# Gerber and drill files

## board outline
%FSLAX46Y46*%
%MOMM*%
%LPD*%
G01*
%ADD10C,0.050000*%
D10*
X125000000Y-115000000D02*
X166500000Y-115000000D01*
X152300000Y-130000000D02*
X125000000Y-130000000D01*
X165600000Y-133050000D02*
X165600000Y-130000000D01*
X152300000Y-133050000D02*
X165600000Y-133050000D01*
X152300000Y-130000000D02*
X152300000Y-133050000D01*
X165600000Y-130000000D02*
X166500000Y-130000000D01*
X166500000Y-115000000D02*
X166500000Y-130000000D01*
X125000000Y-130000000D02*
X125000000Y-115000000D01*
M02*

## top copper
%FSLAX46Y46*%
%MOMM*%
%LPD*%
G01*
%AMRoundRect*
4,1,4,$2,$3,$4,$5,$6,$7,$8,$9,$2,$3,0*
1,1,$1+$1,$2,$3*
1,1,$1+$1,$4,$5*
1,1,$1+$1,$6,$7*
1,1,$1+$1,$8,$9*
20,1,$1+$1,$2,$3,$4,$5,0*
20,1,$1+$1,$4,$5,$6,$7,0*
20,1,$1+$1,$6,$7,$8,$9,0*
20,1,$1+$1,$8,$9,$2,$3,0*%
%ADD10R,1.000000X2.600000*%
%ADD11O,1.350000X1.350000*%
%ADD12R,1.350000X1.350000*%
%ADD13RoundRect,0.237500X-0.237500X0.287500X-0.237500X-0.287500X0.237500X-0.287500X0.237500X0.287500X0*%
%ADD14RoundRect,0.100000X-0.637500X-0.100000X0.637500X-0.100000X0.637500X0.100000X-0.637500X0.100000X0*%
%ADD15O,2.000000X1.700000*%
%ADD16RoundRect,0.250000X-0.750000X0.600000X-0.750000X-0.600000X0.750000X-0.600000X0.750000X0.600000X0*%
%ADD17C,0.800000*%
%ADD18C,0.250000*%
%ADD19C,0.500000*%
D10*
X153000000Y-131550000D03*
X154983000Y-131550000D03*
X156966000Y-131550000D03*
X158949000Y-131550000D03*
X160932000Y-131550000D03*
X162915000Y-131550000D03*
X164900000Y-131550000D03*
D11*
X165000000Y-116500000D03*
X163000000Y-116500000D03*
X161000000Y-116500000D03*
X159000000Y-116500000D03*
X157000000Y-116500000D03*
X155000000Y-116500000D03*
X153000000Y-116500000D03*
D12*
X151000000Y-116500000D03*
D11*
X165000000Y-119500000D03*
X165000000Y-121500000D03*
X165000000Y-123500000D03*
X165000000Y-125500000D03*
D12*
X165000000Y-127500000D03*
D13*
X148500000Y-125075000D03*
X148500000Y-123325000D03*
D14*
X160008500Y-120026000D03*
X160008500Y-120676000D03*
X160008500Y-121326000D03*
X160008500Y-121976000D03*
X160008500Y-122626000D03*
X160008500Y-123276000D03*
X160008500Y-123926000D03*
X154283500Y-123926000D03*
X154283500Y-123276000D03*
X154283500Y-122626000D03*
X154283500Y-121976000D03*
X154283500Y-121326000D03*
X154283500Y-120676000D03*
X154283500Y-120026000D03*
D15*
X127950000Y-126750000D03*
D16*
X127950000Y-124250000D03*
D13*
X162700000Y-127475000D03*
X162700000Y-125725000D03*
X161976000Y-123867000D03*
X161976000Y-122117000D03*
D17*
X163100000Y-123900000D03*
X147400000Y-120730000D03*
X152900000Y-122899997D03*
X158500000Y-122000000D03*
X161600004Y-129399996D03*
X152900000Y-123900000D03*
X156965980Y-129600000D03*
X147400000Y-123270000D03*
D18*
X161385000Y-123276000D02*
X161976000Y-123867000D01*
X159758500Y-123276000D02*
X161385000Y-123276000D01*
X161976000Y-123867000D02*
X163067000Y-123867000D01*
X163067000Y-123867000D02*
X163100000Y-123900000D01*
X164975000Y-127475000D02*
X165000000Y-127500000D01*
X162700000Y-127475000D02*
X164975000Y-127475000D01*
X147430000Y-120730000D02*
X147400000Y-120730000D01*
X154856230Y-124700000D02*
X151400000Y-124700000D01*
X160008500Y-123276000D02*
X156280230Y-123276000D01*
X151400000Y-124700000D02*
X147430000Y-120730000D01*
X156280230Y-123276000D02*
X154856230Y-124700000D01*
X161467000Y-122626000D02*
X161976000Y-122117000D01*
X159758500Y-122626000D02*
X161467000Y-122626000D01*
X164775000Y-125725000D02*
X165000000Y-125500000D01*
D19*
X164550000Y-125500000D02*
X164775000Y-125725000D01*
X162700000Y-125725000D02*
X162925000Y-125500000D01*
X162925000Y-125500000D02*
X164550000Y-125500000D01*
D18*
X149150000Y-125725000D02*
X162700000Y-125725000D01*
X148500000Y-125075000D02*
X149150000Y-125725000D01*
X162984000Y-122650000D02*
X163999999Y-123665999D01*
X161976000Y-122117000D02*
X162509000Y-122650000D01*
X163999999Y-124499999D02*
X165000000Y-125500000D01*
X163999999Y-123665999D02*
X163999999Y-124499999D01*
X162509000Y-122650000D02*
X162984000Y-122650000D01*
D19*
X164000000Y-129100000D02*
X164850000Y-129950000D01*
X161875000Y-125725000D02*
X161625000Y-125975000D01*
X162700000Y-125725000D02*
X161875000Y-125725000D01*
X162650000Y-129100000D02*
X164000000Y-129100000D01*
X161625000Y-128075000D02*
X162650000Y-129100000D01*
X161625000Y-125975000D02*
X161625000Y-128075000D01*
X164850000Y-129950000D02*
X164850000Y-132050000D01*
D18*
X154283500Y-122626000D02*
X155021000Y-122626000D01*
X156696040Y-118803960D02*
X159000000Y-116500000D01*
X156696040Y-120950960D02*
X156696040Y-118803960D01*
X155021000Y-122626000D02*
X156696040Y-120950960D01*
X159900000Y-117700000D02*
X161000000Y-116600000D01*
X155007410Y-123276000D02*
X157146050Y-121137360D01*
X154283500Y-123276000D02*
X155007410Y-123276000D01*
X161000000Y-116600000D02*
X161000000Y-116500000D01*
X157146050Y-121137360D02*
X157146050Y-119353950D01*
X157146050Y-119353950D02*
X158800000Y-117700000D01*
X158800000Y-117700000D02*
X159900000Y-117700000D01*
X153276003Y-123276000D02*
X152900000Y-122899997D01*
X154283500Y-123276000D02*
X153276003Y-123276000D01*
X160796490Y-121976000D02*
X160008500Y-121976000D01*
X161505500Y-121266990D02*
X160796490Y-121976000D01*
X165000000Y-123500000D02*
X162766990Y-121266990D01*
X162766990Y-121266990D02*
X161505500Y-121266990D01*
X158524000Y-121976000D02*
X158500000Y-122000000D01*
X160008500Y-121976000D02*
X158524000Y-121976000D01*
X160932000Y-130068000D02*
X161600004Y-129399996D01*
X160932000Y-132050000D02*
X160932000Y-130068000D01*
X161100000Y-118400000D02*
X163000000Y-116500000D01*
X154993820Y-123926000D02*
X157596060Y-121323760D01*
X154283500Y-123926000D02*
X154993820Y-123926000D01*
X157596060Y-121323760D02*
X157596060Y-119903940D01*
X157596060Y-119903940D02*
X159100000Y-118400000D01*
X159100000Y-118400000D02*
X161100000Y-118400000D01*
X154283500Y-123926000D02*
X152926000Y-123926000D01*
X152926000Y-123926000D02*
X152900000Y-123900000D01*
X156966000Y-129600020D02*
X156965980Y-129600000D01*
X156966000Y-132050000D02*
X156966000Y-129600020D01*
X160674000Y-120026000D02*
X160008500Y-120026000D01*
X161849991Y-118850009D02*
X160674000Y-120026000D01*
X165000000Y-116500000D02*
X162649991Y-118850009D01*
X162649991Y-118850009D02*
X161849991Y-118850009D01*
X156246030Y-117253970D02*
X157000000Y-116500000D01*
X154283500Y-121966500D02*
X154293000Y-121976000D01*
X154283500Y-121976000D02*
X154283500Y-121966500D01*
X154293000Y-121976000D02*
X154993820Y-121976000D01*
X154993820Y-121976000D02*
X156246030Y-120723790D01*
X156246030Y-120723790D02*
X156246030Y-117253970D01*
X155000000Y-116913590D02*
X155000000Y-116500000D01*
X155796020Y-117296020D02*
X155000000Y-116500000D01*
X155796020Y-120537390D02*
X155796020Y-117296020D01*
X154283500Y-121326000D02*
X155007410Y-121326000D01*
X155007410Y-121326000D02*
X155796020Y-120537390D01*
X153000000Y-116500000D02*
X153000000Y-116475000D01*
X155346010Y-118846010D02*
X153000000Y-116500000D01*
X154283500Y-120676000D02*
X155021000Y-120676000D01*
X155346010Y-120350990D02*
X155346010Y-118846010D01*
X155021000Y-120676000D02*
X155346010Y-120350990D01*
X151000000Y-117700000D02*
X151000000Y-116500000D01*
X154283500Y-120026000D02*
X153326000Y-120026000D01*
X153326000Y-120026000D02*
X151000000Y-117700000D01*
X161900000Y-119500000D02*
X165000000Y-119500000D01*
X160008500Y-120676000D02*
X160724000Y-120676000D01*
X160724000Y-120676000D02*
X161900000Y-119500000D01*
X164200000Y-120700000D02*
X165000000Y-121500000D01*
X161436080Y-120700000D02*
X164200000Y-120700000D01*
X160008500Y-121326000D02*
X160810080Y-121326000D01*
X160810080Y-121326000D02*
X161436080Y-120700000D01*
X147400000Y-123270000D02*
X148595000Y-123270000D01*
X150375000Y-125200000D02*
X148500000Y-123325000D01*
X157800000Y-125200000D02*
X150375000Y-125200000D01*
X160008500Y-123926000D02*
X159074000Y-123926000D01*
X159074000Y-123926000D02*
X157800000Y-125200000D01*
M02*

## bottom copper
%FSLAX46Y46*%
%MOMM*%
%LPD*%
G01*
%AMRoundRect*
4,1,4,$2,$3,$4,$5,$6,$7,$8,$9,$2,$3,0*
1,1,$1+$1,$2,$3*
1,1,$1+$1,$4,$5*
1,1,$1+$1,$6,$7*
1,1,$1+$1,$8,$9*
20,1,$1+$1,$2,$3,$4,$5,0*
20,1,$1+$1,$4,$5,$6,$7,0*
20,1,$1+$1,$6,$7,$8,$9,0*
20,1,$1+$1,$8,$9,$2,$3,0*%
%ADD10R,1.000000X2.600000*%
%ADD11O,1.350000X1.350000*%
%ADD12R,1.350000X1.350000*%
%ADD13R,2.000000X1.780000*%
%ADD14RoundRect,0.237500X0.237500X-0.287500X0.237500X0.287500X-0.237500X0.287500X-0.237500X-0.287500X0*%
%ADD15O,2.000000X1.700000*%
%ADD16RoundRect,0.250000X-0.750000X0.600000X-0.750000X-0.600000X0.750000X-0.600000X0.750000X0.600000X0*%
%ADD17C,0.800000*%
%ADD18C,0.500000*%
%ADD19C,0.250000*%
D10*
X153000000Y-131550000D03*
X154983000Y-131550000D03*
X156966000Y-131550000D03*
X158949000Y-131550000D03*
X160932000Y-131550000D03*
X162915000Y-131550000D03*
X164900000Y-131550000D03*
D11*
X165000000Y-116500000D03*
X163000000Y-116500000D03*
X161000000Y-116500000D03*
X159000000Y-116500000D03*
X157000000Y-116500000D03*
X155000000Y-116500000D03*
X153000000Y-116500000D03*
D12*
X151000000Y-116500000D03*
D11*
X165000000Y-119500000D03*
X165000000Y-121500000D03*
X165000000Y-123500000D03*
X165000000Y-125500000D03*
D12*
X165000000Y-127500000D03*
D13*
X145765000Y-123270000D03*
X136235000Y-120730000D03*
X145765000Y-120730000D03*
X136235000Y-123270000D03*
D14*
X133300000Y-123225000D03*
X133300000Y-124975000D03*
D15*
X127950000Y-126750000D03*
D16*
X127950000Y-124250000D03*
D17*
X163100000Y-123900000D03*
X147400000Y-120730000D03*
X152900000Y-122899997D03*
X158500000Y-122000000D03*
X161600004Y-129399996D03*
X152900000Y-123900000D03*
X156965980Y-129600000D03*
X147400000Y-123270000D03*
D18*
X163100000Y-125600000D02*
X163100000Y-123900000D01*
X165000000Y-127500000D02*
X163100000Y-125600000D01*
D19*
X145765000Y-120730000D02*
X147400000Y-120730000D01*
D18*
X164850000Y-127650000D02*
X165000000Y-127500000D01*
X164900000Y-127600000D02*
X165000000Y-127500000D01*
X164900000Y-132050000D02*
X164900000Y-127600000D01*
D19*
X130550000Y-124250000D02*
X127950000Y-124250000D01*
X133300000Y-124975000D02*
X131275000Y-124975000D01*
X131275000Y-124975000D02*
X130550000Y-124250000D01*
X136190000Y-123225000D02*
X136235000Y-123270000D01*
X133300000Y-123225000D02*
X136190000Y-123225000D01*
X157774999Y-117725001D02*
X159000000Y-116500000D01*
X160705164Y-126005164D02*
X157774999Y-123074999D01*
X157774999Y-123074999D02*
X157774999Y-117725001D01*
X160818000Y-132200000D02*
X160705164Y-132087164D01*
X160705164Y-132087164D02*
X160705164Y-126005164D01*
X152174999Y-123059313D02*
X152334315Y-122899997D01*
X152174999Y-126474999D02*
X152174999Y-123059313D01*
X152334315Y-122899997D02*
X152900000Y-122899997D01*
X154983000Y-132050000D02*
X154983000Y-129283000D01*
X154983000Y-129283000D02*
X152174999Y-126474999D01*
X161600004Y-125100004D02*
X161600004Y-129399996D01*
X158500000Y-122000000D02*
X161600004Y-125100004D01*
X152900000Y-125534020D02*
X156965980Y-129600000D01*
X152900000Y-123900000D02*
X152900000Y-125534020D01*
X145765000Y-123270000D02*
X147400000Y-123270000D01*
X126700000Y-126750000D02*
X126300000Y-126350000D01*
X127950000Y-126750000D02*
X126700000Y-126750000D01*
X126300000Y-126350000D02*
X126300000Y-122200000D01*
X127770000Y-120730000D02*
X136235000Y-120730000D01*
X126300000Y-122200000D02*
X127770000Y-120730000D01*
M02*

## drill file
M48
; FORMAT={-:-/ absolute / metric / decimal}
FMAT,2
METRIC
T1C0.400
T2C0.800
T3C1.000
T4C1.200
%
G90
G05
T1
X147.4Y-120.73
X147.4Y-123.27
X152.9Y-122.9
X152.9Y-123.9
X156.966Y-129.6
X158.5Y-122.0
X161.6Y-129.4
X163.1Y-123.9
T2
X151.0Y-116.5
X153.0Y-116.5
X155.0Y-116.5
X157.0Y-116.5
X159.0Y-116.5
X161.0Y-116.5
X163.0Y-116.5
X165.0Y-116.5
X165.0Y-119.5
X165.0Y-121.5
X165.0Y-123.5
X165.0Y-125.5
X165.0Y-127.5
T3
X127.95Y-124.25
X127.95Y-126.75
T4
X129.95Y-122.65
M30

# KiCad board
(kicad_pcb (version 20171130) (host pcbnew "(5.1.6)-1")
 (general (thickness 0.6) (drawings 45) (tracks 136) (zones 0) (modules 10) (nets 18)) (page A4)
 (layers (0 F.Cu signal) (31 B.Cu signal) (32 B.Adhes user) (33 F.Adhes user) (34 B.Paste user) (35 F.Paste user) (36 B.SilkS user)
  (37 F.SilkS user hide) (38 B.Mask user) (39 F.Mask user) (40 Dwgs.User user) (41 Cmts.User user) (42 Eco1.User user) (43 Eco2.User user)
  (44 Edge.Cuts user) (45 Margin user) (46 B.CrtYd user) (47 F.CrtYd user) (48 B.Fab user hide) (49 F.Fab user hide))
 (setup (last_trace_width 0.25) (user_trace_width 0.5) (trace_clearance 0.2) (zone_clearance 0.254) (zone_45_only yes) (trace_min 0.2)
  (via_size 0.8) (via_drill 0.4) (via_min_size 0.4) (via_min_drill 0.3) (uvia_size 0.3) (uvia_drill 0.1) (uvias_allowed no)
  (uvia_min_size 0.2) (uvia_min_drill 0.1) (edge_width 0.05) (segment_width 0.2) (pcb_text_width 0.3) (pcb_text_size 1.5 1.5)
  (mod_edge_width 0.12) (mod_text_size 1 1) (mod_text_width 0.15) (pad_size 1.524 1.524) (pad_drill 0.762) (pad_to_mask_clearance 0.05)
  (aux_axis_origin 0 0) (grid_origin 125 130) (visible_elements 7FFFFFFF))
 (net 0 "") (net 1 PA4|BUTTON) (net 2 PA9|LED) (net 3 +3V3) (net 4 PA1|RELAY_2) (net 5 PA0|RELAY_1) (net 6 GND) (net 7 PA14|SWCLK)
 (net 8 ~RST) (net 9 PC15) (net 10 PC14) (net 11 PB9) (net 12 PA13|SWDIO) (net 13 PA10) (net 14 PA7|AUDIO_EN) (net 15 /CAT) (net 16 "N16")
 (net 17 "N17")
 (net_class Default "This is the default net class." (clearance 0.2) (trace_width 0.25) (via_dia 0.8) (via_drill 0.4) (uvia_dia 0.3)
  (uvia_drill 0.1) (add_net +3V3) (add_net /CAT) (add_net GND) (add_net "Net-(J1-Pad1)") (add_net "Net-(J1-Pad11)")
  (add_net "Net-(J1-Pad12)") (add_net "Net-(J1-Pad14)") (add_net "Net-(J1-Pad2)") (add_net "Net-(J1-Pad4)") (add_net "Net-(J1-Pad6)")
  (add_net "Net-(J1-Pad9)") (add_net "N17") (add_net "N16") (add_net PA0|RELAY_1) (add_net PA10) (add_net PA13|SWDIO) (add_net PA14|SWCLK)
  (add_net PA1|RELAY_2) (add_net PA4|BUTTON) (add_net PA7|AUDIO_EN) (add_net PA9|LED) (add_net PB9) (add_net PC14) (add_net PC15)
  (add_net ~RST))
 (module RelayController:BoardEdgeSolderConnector (layer F.Cu) (at 153 131.55)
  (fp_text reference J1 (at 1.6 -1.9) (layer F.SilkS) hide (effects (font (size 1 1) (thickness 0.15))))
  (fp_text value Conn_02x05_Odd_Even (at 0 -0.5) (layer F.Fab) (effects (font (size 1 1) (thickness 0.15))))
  (pad 1 smd rect (at 0 0) (size 1 2.6) (layers F.Cu F.Paste F.Mask))
  (pad 2 smd rect (at 1.983 0) (size 1 2.6) (layers F.Cu F.Paste F.Mask))
  (pad 3 smd rect (at 3.966 0) (size 1 2.6) (layers F.Cu F.Paste F.Mask) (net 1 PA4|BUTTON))
  (pad 4 smd rect (at 5.949 0) (size 1 2.6) (layers F.Cu F.Paste F.Mask))
  (pad 5 smd rect (at 7.932 0) (size 1 2.6) (layers F.Cu F.Paste F.Mask) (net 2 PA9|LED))
  (pad 6 smd rect (at 9.915 0) (size 1 2.6) (layers F.Cu F.Paste F.Mask))
  (pad 7 smd rect (at 11.9 0) (size 1 2.6) (layers F.Cu F.Paste F.Mask) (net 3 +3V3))
  (pad 14 smd rect (at 0 0) (size 1 2.6) (layers B.Cu B.Paste B.Mask))
  (pad 13 smd rect (at 1.983 0) (size 1 2.6) (layers B.Cu B.Paste B.Mask) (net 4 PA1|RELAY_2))
  (pad 12 smd rect (at 3.966 0) (size 1 2.6) (layers B.Cu B.Paste B.Mask))
  (pad 11 smd rect (at 5.949 0) (size 1 2.6) (layers B.Cu B.Paste B.Mask))
  (pad 10 smd rect (at 7.932 0) (size 1 2.6) (layers B.Cu B.Paste B.Mask) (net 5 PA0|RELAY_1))
  (pad 9 smd rect (at 9.915 0) (size 1 2.6) (layers B.Cu B.Paste B.Mask))
  (pad 8 smd rect (at 11.9 0) (size 1 2.6) (layers B.Cu B.Paste B.Mask) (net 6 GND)))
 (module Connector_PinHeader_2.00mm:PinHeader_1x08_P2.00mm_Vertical (layer F.Cu) (at 151 116.5 90)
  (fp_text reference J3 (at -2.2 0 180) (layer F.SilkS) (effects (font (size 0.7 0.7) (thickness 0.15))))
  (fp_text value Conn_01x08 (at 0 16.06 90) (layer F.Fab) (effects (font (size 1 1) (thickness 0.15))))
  (pad 8 thru_hole oval (at 0 14 90) (size 1.35 1.35) (drill 0.8) (layers *.Cu *.Mask) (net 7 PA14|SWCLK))
  (pad 7 thru_hole oval (at 0 12 90) (size 1.35 1.35) (drill 0.8) (layers *.Cu *.Mask) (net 1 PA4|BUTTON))
  (pad 6 thru_hole oval (at 0 10 90) (size 1.35 1.35) (drill 0.8) (layers *.Cu *.Mask) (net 4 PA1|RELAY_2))
  (pad 5 thru_hole oval (at 0 8 90) (size 1.35 1.35) (drill 0.8) (layers *.Cu *.Mask) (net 5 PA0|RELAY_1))
  (pad 4 thru_hole oval (at 0 6 90) (size 1.35 1.35) (drill 0.8) (layers *.Cu *.Mask) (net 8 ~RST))
  (pad 3 thru_hole oval (at 0 4 90) (size 1.35 1.35) (drill 0.8) (layers *.Cu *.Mask) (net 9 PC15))
  (pad 2 thru_hole oval (at 0 2 90) (size 1.35 1.35) (drill 0.8) (layers *.Cu *.Mask) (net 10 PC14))
  (pad 1 thru_hole rect (at 0 0 90) (size 1.35 1.35) (drill 0.8) (layers *.Cu *.Mask) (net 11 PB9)))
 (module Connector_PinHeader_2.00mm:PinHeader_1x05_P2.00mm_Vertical (layer F.Cu) (at 165 127.5 180)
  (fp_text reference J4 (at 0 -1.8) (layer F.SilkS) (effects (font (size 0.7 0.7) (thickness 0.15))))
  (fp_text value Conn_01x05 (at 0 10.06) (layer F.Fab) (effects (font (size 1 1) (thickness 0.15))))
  (pad 5 thru_hole oval (at 0 8 180) (size 1.35 1.35) (drill 0.8) (layers *.Cu *.Mask) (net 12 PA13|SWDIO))
  (pad 4 thru_hole oval (at 0 6 180) (size 1.35 1.35) (drill 0.8) (layers *.Cu *.Mask) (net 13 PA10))
  (pad 3 thru_hole oval (at 0 4 180) (size 1.35 1.35) (drill 0.8) (layers *.Cu *.Mask) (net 2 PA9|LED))
  (pad 2 thru_hole oval (at 0 2 180) (size 1.35 1.35) (drill 0.8) (layers *.Cu *.Mask) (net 3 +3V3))
  (pad 1 thru_hole rect (at 0 0 180) (size 1.35 1.35) (drill 0.8) (layers *.Cu *.Mask) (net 6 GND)))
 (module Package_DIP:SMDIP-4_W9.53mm (layer B.Cu) (at 141 122)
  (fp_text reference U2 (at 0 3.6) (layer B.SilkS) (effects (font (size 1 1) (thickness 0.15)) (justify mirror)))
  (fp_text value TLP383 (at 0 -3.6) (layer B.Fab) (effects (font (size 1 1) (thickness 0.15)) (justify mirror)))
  (pad 4 smd rect (at 4.765 1.27) (size 2 1.78) (layers B.Cu B.Paste B.Mask) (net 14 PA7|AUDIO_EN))
  (pad 2 smd rect (at -4.765 -1.27) (size 2 1.78) (layers B.Cu B.Paste B.Mask) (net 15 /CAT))
  (pad 3 smd rect (at 4.765 -1.27) (size 2 1.78) (layers B.Cu B.Paste B.Mask) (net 6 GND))
  (pad 1 smd rect (at -4.765 1.27) (size 2 1.78) (layers B.Cu B.Paste B.Mask) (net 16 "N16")))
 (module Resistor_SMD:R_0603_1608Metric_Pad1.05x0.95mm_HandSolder (layer F.Cu) (at 148.5 124.2 270)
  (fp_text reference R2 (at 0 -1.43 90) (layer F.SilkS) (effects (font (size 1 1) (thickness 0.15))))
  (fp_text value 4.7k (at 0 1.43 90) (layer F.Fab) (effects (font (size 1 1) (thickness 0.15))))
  (pad 2 smd roundrect (at 0.875 0 270) (size 1.05 0.95) (layers F.Cu F.Paste F.Mask) (roundrect_rratio 0.25) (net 3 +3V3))
  (pad 1 smd roundrect (at -0.875 0 270) (size 1.05 0.95) (layers F.Cu F.Paste F.Mask) (roundrect_rratio 0.25) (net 14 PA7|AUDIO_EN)))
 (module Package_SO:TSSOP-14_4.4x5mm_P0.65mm (layer F.Cu) (at 157.146 121.976)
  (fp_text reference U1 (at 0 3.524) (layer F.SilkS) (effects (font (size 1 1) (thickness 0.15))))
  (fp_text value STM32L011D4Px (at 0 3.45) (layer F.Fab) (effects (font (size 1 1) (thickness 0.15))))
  (pad 14 smd roundrect (at 2.8625 -1.95) (size 1.475 0.4) (layers F.Cu F.Paste F.Mask) (roundrect_rratio 0.25) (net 7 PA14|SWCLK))
  (pad 13 smd roundrect (at 2.8625 -1.3) (size 1.475 0.4) (layers F.Cu F.Paste F.Mask) (roundrect_rratio 0.25) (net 12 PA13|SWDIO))
  (pad 12 smd roundrect (at 2.8625 -0.65) (size 1.475 0.4) (layers F.Cu F.Paste F.Mask) (roundrect_rratio 0.25) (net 13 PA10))
  (pad 11 smd roundrect (at 2.8625 0) (size 1.475 0.4) (layers F.Cu F.Paste F.Mask) (roundrect_rratio 0.25) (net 2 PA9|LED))
  (pad 10 smd roundrect (at 2.8625 0.65) (size 1.475 0.4) (layers F.Cu F.Paste F.Mask) (roundrect_rratio 0.25) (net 3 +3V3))
  (pad 9 smd roundrect (at 2.8625 1.3) (size 1.475 0.4) (layers F.Cu F.Paste F.Mask) (roundrect_rratio 0.25) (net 6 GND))
  (pad 8 smd roundrect (at 2.8625 1.95) (size 1.475 0.4) (layers F.Cu F.Paste F.Mask) (roundrect_rratio 0.25) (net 14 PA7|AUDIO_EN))
  (pad 7 smd roundrect (at -2.8625 1.95) (size 1.475 0.4) (layers F.Cu F.Paste F.Mask) (roundrect_rratio 0.25) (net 1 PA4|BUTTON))
  (pad 6 smd roundrect (at -2.8625 1.3) (size 1.475 0.4) (layers F.Cu F.Paste F.Mask) (roundrect_rratio 0.25) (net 4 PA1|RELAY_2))
  (pad 5 smd roundrect (at -2.8625 0.65) (size 1.475 0.4) (layers F.Cu F.Paste F.Mask) (roundrect_rratio 0.25) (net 5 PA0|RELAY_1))
  (pad 4 smd roundrect (at -2.8625 0) (size 1.475 0.4) (layers F.Cu F.Paste F.Mask) (roundrect_rratio 0.25) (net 8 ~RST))
  (pad 3 smd roundrect (at -2.8625 -0.65) (size 1.475 0.4) (layers F.Cu F.Paste F.Mask) (roundrect_rratio 0.25) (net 9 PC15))
  (pad 2 smd roundrect (at -2.8625 -1.3) (size 1.475 0.4) (layers F.Cu F.Paste F.Mask) (roundrect_rratio 0.25) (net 10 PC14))
  (pad 1 smd roundrect (at -2.8625 -1.95) (size 1.475 0.4) (layers F.Cu F.Paste F.Mask) (roundrect_rratio 0.25) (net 11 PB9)))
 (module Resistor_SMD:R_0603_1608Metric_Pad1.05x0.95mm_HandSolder (layer B.Cu) (at 133.3 124.1 90)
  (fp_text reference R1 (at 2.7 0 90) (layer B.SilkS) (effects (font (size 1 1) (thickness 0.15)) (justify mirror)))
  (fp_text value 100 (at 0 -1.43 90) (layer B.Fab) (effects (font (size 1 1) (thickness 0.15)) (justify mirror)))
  (pad 2 smd roundrect (at 0.875 0 90) (size 1.05 0.95) (layers B.Cu B.Paste B.Mask) (roundrect_rratio 0.25) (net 16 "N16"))
  (pad 1 smd roundrect (at -0.875 0 90) (size 1.05 0.95) (layers B.Cu B.Paste B.Mask) (roundrect_rratio 0.25) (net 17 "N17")))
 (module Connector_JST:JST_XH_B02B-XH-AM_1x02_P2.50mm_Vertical (layer B.Cu) (at 127.95 124.25 270)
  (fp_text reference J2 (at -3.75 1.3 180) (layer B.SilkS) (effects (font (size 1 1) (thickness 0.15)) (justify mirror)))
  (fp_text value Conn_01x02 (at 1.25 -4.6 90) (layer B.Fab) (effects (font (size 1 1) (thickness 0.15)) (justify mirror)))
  (pad "" np_thru_hole circle (at -1.6 -2 270) (size 1.2 1.2) (drill 1.2) (layers *.Cu *.Mask))
  (pad 2 thru_hole oval (at 2.5 0 270) (size 1.7 2) (drill 1) (layers *.Cu *.Mask) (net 15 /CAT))
  (pad 1 thru_hole roundrect (at 0 0 270) (size 1.7 2) (drill 1) (layers *.Cu *.Mask) (roundrect_rratio 0.147059) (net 17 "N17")))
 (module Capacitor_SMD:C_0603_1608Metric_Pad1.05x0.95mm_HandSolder (layer F.Cu) (at 162.7 126.6 270)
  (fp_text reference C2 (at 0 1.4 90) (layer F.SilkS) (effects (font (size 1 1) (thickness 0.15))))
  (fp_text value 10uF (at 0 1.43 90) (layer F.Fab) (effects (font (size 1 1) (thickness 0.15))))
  (pad 2 smd roundrect (at 0.875 0 270) (size 1.05 0.95) (layers F.Cu F.Paste F.Mask) (roundrect_rratio 0.25) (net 6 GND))
  (pad 1 smd roundrect (at -0.875 0 270) (size 1.05 0.95) (layers F.Cu F.Paste F.Mask) (roundrect_rratio 0.25) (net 3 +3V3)))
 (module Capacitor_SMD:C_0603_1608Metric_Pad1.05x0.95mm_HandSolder (layer F.Cu) (at 161.976 122.992 270)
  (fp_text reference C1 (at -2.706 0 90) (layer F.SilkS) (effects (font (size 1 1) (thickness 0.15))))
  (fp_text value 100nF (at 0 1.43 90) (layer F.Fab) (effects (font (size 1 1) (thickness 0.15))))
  (pad 2 smd roundrect (at 0.875 0 270) (size 1.05 0.95) (layers F.Cu F.Paste F.Mask) (roundrect_rratio 0.25) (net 6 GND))
  (pad 1 smd roundrect (at -0.875 0 270) (size 1.05 0.95) (layers F.Cu F.Paste F.Mask) (roundrect_rratio 0.25) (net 3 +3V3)))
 (gr_line (start 125 115) (end 166.5 115) (layer Edge.Cuts) (width 0.05))
 (gr_line (start 152.3 130) (end 125 130) (layer Edge.Cuts) (width 0.05))
 (gr_line (start 165.6 133.05) (end 165.6 130) (layer Edge.Cuts) (width 0.05))
 (gr_line (start 152.3 133.05) (end 165.6 133.05) (layer Edge.Cuts) (width 0.05))
 (gr_line (start 152.3 130) (end 152.3 133.05) (layer Edge.Cuts) (width 0.05))
 (gr_line (start 165.6 130) (end 166.5 130) (layer Edge.Cuts) (width 0.05))
 (gr_line (start 166.5 115) (end 166.5 130) (layer Edge.Cuts) (width 0.05))
 (gr_line (start 125 130) (end 125 115) (layer Edge.Cuts) (width 0.05))
 (segment (start 161.385 123.276) (end 161.976 123.867) (width 0.25) (layer F.Cu) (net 6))
 (segment (start 159.7585 123.276) (end 161.385 123.276) (width 0.25) (layer F.Cu) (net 6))
 (via (at 163.1 123.9) (size 0.8) (drill 0.4) (layers F.Cu B.Cu) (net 6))
 (segment (start 161.976 123.867) (end 163.067 123.867) (width 0.25) (layer F.Cu) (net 6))
 (segment (start 163.067 123.867) (end 163.1 123.9) (width 0.25) (layer F.Cu) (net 6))
 (segment (start 164.975 127.475) (end 165 127.5) (width 0.25) (layer F.Cu) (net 6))
 (segment (start 162.7 127.475) (end 164.975 127.475) (width 0.25) (layer F.Cu) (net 6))
 (segment (start 163.1 125.6) (end 163.1 123.9) (width 0.5) (layer B.Cu) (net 6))
 (segment (start 165 127.5) (end 163.1 125.6) (width 0.5) (layer B.Cu) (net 6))
 (segment (start 145.765 120.73) (end 147.4 120.73) (width 0.25) (layer B.Cu) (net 6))
 (via (at 147.4 120.73) (size 0.8) (drill 0.4) (layers F.Cu B.Cu) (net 6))
 (segment (start 147.43 120.73) (end 147.4 120.73) (width 0.25) (layer F.Cu) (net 6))
 (segment (start 154.85623 124.7) (end 151.4 124.7) (width 0.25) (layer F.Cu) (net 6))
 (segment (start 160.0085 123.276) (end 156.28023 123.276) (width 0.25) (layer F.Cu) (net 6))
 (segment (start 151.4 124.7) (end 147.43 120.73) (width 0.25) (layer F.Cu) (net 6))
 (segment (start 156.28023 123.276) (end 154.85623 124.7) (width 0.25) (layer F.Cu) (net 6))
 (segment (start 164.85 127.65) (end 165 127.5) (width 0.5) (layer B.Cu) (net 6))
 (segment (start 164.9 127.6) (end 165 127.5) (width 0.5) (layer B.Cu) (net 6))
 (segment (start 164.9 132.05) (end 164.9 127.6) (width 0.5) (layer B.Cu) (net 6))
 (segment (start 161.467 122.626) (end 161.976 122.117) (width 0.25) (layer F.Cu) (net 3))
 (segment (start 159.7585 122.626) (end 161.467 122.626) (width 0.25) (layer F.Cu) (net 3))
 (segment (start 164.775 125.725) (end 165 125.5) (width 0.25) (layer F.Cu) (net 3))
 (segment (start 164.55 125.5) (end 164.775 125.725) (width 0.5) (layer F.Cu) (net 3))
 (segment (start 162.7 125.725) (end 162.925 125.5) (width 0.5) (layer F.Cu) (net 3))
 (segment (start 162.925 125.5) (end 164.55 125.5) (width 0.5) (layer F.Cu) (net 3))
 (segment (start 149.15 125.725) (end 162.7 125.725) (width 0.25) (layer F.Cu) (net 3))
 (segment (start 148.5 125.075) (end 149.15 125.725) (width 0.25) (layer F.Cu) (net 3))
 (segment (start 162.984 122.65) (end 163.999999 123.665999) (width 0.25) (layer F.Cu) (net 3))
 (segment (start 161.976 122.117) (end 162.509 122.65) (width 0.25) (layer F.Cu) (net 3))
 (segment (start 163.999999 124.499999) (end 165 125.5) (width 0.25) (layer F.Cu) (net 3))
 (segment (start 163.999999 123.665999) (end 163.999999 124.499999) (width 0.25) (layer F.Cu) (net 3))
 (segment (start 162.509 122.65) (end 162.984 122.65) (width 0.25) (layer F.Cu) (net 3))
 (segment (start 164 129.1) (end 164.85 129.95) (width 0.5) (layer F.Cu) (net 3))
 (segment (start 161.875 125.725) (end 161.625 125.975) (width 0.5) (layer F.Cu) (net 3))
 (segment (start 162.7 125.725) (end 161.875 125.725) (width 0.5) (layer F.Cu) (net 3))
 (segment (start 162.65 129.1) (end 164 129.1) (width 0.5) (layer F.Cu) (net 3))
 (segment (start 161.625 128.075) (end 162.65 129.1) (width 0.5) (layer F.Cu) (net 3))
 (segment (start 161.625 125.975) (end 161.625 128.075) (width 0.5) (layer F.Cu) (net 3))
 (segment (start 164.85 129.95) (end 164.85 132.05) (width 0.5) (layer F.Cu) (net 3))
 (segment (start 130.55 124.25) (end 127.95 124.25) (width 0.25) (layer B.Cu) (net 17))
 (segment (start 133.3 124.975) (end 131.275 124.975) (width 0.25) (layer B.Cu) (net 17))
 (segment (start 131.275 124.975) (end 130.55 124.25) (width 0.25) (layer B.Cu) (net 17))
 (segment (start 136.19 123.225) (end 136.235 123.27) (width 0.25) (layer B.Cu) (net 16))
 (segment (start 133.3 123.225) (end 136.19 123.225) (width 0.25) (layer B.Cu) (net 16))
 (segment (start 154.2835 122.626) (end 155.021 122.626) (width 0.25) (layer F.Cu) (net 5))
 (segment (start 156.69604 118.80396) (end 159 116.5) (width 0.25) (layer F.Cu) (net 5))
 (segment (start 156.69604 120.95096) (end 156.69604 118.80396) (width 0.25) (layer F.Cu) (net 5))
 (segment (start 155.021 122.626) (end 156.69604 120.95096) (width 0.25) (layer F.Cu) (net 5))
 (segment (start 157.774999 117.725001) (end 159 116.5) (width 0.25) (layer B.Cu) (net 5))
 (segment (start 160.705164 126.005164) (end 157.774999 123.074999) (width 0.25) (layer B.Cu) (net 5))
 (segment (start 157.774999 123.074999) (end 157.774999 117.725001) (width 0.25) (layer B.Cu) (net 5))
 (segment (start 160.818 132.2) (end 160.705164 132.087164) (width 0.25) (layer B.Cu) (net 5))
 (segment (start 160.705164 132.087164) (end 160.705164 126.005164) (width 0.25) (layer B.Cu) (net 5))
 (segment (start 159.9 117.7) (end 161 116.6) (width 0.25) (layer F.Cu) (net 4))
 (segment (start 155.00741 123.276) (end 157.14605 121.13736) (width 0.25) (layer F.Cu) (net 4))
 (segment (start 154.2835 123.276) (end 155.00741 123.276) (width 0.25) (layer F.Cu) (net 4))
 (segment (start 161 116.6) (end 161 116.5) (width 0.25) (layer F.Cu) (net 4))
 (segment (start 157.14605 121.13736) (end 157.14605 119.35395) (width 0.25) (layer F.Cu) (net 4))
 (segment (start 157.14605 119.35395) (end 158.8 117.7) (width 0.25) (layer F.Cu) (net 4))
 (segment (start 158.8 117.7) (end 159.9 117.7) (width 0.25) (layer F.Cu) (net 4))
 (segment (start 153.276003 123.276) (end 152.9 122.899997) (width 0.25) (layer F.Cu) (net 4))
 (segment (start 154.2835 123.276) (end 153.276003 123.276) (width 0.25) (layer F.Cu) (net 4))
 (via (at 152.9 122.899997) (size 0.8) (drill 0.4) (layers F.Cu B.Cu) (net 4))
 (segment (start 152.174999 123.059313) (end 152.334315 122.899997) (width 0.25) (layer B.Cu) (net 4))
 (segment (start 152.174999 126.474999) (end 152.174999 123.059313) (width 0.25) (layer B.Cu) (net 4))
 (segment (start 152.334315 122.899997) (end 152.9 122.899997) (width 0.25) (layer B.Cu) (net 4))
 (segment (start 154.983 132.05) (end 154.983 129.283) (width 0.25) (layer B.Cu) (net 4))
 (segment (start 154.983 129.283) (end 152.174999 126.474999) (width 0.25) (layer B.Cu) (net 4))
 (segment (start 160.79649 121.976) (end 160.0085 121.976) (width 0.25) (layer F.Cu) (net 2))
 (segment (start 161.5055 121.26699) (end 160.79649 121.976) (width 0.25) (layer F.Cu) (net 2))
 (segment (start 165 123.5) (end 162.76699 121.26699) (width 0.25) (layer F.Cu) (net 2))
 (segment (start 162.76699 121.26699) (end 161.5055 121.26699) (width 0.25) (layer F.Cu) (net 2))
 (via (at 158.5 122) (size 0.8) (drill 0.4) (layers F.Cu B.Cu) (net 2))
 (segment (start 158.524 121.976) (end 158.5 122) (width 0.25) (layer F.Cu) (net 2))
 (segment (start 160.0085 121.976) (end 158.524 121.976) (width 0.25) (layer F.Cu) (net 2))
 (via (at 161.600004 129.399996) (size 0.8) (drill 0.4) (layers F.Cu B.Cu) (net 2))
 (segment (start 161.600004 125.100004) (end 161.600004 129.399996) (width 0.25) (layer B.Cu) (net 2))
 (segment (start 158.5 122) (end 161.600004 125.100004) (width 0.25) (layer B.Cu) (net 2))
 (segment (start 160.932 130.068) (end 161.600004 129.399996) (width 0.25) (layer F.Cu) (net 2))
 (segment (start 160.932 132.05) (end 160.932 130.068) (width 0.25) (layer F.Cu) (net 2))
 (segment (start 161.1 118.4) (end 163 116.5) (width 0.25) (layer F.Cu) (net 1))
 (segment (start 154.99382 123.926) (end 157.59606 121.32376) (width 0.25) (layer F.Cu) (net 1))
 (segment (start 154.2835 123.926) (end 154.99382 123.926) (width 0.25) (layer F.Cu) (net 1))
 (segment (start 157.59606 121.32376) (end 157.59606 119.90394) (width 0.25) (layer F.Cu) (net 1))
 (segment (start 157.59606 119.90394) (end 159.1 118.4) (width 0.25) (layer F.Cu) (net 1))
 (segment (start 159.1 118.4) (end 161.1 118.4) (width 0.25) (layer F.Cu) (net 1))
 (via (at 152.9 123.9) (size 0.8) (drill 0.4) (layers F.Cu B.Cu) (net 1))
 (segment (start 154.2835 123.926) (end 152.926 123.926) (width 0.25) (layer F.Cu) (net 1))
 (segment (start 152.926 123.926) (end 152.9 123.9) (width 0.25) (layer F.Cu) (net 1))
 (via (at 156.96598 129.6) (size 0.8) (drill 0.4) (layers F.Cu B.Cu) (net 1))
 (segment (start 156.966 129.60002) (end 156.96598 129.6) (width 0.25) (layer F.Cu) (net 1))
 (segment (start 156.966 132.05) (end 156.966 129.60002) (width 0.25) (layer F.Cu) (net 1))
 (segment (start 152.9 125.53402) (end 156.96598 129.6) (width 0.25) (layer B.Cu) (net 1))
 (segment (start 152.9 123.9) (end 152.9 125.53402) (width 0.25) (layer B.Cu) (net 1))
 (segment (start 160.674 120.026) (end 160.0085 120.026) (width 0.25) (layer F.Cu) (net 7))
 (segment (start 161.849991 118.850009) (end 160.674 120.026) (width 0.25) (layer F.Cu) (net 7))
 (segment (start 165 116.5) (end 162.649991 118.850009) (width 0.25) (layer F.Cu) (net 7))
 (segment (start 162.649991 118.850009) (end 161.849991 118.850009) (width 0.25) (layer F.Cu) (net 7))
 (segment (start 156.24603 117.25397) (end 157 116.5) (width 0.25) (layer F.Cu) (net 8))
 (segment (start 154.2835 121.9665) (end 154.293 121.976) (width 0.25) (layer F.Cu) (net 8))
 (segment (start 154.2835 121.976) (end 154.2835 121.9665) (width 0.25) (layer F.Cu) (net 8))
 (segment (start 154.293 121.976) (end 154.99382 121.976) (width 0.25) (layer F.Cu) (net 8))
 (segment (start 154.99382 121.976) (end 156.24603 120.72379) (width 0.25) (layer F.Cu) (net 8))
 (segment (start 156.24603 120.72379) (end 156.24603 117.25397) (width 0.25) (layer F.Cu) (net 8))
 (segment (start 155 116.91359) (end 155 116.5) (width 0.25) (layer F.Cu) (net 9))
 (segment (start 155.79602 117.29602) (end 155 116.5) (width 0.25) (layer F.Cu) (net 9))
 (segment (start 155.79602 120.53739) (end 155.79602 117.29602) (width 0.25) (layer F.Cu) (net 9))
 (segment (start 154.2835 121.326) (end 155.00741 121.326) (width 0.25) (layer F.Cu) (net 9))
 (segment (start 155.00741 121.326) (end 155.79602 120.53739) (width 0.25) (layer F.Cu) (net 9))
 (segment (start 153 116.5) (end 153 116.475) (width 0.25) (layer F.Cu) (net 10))
 (segment (start 155.34601 118.84601) (end 153 116.5) (width 0.25) (layer F.Cu) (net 10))
 (segment (start 154.2835 120.676) (end 155.021 120.676) (width 0.25) (layer F.Cu) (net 10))
 (segment (start 155.34601 120.35099) (end 155.34601 118.84601) (width 0.25) (layer F.Cu) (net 10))
 (segment (start 155.021 120.676) (end 155.34601 120.35099) (width 0.25) (layer F.Cu) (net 10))
 (segment (start 151 117.7) (end 151 116.5) (width 0.25) (layer F.Cu) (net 11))
 (segment (start 154.2835 120.026) (end 153.326 120.026) (width 0.25) (layer F.Cu) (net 11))
 (segment (start 153.326 120.026) (end 151 117.7) (width 0.25) (layer F.Cu) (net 11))
 (segment (start 161.9 119.5) (end 165 119.5) (width 0.25) (layer F.Cu) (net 12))
 (segment (start 160.0085 120.676) (end 160.724 120.676) (width 0.25) (layer F.Cu) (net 12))
 (segment (start 160.724 120.676) (end 161.9 119.5) (width 0.25) (layer F.Cu) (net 12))
 (segment (start 164.2 120.7) (end 165 121.5) (width 0.25) (layer F.Cu) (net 13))
 (segment (start 161.43608 120.7) (end 164.2 120.7) (width 0.25) (layer F.Cu) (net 13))
 (segment (start 160.0085 121.326) (end 160.81008 121.326) (width 0.25) (layer F.Cu) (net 13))
 (segment (start 160.81008 121.326) (end 161.43608 120.7) (width 0.25) (layer F.Cu) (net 13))
 (via (at 147.4 123.27) (size 0.8) (drill 0.4) (layers F.Cu B.Cu) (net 14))
 (segment (start 145.765 123.27) (end 147.4 123.27) (width 0.25) (layer B.Cu) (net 14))
 (segment (start 147.4 123.27) (end 148.595 123.27) (width 0.25) (layer F.Cu) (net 14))
 (segment (start 150.375 125.2) (end 148.5 123.325) (width 0.25) (layer F.Cu) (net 14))
 (segment (start 157.8 125.2) (end 150.375 125.2) (width 0.25) (layer F.Cu) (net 14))
 (segment (start 160.0085 123.926) (end 159.074 123.926) (width 0.25) (layer F.Cu) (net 14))
 (segment (start 159.074 123.926) (end 157.8 125.2) (width 0.25) (layer F.Cu) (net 14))
 (segment (start 126.7 126.75) (end 126.3 126.35) (width 0.25) (layer B.Cu) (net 15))
 (segment (start 127.95 126.75) (end 126.7 126.75) (width 0.25) (layer B.Cu) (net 15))
 (segment (start 126.3 126.35) (end 126.3 122.2) (width 0.25) (layer B.Cu) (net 15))
 (segment (start 127.77 120.73) (end 136.235 120.73) (width 0.25) (layer B.Cu) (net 15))
 (segment (start 126.3 122.2) (end 127.77 120.73) (width 0.25) (layer B.Cu) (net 15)))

